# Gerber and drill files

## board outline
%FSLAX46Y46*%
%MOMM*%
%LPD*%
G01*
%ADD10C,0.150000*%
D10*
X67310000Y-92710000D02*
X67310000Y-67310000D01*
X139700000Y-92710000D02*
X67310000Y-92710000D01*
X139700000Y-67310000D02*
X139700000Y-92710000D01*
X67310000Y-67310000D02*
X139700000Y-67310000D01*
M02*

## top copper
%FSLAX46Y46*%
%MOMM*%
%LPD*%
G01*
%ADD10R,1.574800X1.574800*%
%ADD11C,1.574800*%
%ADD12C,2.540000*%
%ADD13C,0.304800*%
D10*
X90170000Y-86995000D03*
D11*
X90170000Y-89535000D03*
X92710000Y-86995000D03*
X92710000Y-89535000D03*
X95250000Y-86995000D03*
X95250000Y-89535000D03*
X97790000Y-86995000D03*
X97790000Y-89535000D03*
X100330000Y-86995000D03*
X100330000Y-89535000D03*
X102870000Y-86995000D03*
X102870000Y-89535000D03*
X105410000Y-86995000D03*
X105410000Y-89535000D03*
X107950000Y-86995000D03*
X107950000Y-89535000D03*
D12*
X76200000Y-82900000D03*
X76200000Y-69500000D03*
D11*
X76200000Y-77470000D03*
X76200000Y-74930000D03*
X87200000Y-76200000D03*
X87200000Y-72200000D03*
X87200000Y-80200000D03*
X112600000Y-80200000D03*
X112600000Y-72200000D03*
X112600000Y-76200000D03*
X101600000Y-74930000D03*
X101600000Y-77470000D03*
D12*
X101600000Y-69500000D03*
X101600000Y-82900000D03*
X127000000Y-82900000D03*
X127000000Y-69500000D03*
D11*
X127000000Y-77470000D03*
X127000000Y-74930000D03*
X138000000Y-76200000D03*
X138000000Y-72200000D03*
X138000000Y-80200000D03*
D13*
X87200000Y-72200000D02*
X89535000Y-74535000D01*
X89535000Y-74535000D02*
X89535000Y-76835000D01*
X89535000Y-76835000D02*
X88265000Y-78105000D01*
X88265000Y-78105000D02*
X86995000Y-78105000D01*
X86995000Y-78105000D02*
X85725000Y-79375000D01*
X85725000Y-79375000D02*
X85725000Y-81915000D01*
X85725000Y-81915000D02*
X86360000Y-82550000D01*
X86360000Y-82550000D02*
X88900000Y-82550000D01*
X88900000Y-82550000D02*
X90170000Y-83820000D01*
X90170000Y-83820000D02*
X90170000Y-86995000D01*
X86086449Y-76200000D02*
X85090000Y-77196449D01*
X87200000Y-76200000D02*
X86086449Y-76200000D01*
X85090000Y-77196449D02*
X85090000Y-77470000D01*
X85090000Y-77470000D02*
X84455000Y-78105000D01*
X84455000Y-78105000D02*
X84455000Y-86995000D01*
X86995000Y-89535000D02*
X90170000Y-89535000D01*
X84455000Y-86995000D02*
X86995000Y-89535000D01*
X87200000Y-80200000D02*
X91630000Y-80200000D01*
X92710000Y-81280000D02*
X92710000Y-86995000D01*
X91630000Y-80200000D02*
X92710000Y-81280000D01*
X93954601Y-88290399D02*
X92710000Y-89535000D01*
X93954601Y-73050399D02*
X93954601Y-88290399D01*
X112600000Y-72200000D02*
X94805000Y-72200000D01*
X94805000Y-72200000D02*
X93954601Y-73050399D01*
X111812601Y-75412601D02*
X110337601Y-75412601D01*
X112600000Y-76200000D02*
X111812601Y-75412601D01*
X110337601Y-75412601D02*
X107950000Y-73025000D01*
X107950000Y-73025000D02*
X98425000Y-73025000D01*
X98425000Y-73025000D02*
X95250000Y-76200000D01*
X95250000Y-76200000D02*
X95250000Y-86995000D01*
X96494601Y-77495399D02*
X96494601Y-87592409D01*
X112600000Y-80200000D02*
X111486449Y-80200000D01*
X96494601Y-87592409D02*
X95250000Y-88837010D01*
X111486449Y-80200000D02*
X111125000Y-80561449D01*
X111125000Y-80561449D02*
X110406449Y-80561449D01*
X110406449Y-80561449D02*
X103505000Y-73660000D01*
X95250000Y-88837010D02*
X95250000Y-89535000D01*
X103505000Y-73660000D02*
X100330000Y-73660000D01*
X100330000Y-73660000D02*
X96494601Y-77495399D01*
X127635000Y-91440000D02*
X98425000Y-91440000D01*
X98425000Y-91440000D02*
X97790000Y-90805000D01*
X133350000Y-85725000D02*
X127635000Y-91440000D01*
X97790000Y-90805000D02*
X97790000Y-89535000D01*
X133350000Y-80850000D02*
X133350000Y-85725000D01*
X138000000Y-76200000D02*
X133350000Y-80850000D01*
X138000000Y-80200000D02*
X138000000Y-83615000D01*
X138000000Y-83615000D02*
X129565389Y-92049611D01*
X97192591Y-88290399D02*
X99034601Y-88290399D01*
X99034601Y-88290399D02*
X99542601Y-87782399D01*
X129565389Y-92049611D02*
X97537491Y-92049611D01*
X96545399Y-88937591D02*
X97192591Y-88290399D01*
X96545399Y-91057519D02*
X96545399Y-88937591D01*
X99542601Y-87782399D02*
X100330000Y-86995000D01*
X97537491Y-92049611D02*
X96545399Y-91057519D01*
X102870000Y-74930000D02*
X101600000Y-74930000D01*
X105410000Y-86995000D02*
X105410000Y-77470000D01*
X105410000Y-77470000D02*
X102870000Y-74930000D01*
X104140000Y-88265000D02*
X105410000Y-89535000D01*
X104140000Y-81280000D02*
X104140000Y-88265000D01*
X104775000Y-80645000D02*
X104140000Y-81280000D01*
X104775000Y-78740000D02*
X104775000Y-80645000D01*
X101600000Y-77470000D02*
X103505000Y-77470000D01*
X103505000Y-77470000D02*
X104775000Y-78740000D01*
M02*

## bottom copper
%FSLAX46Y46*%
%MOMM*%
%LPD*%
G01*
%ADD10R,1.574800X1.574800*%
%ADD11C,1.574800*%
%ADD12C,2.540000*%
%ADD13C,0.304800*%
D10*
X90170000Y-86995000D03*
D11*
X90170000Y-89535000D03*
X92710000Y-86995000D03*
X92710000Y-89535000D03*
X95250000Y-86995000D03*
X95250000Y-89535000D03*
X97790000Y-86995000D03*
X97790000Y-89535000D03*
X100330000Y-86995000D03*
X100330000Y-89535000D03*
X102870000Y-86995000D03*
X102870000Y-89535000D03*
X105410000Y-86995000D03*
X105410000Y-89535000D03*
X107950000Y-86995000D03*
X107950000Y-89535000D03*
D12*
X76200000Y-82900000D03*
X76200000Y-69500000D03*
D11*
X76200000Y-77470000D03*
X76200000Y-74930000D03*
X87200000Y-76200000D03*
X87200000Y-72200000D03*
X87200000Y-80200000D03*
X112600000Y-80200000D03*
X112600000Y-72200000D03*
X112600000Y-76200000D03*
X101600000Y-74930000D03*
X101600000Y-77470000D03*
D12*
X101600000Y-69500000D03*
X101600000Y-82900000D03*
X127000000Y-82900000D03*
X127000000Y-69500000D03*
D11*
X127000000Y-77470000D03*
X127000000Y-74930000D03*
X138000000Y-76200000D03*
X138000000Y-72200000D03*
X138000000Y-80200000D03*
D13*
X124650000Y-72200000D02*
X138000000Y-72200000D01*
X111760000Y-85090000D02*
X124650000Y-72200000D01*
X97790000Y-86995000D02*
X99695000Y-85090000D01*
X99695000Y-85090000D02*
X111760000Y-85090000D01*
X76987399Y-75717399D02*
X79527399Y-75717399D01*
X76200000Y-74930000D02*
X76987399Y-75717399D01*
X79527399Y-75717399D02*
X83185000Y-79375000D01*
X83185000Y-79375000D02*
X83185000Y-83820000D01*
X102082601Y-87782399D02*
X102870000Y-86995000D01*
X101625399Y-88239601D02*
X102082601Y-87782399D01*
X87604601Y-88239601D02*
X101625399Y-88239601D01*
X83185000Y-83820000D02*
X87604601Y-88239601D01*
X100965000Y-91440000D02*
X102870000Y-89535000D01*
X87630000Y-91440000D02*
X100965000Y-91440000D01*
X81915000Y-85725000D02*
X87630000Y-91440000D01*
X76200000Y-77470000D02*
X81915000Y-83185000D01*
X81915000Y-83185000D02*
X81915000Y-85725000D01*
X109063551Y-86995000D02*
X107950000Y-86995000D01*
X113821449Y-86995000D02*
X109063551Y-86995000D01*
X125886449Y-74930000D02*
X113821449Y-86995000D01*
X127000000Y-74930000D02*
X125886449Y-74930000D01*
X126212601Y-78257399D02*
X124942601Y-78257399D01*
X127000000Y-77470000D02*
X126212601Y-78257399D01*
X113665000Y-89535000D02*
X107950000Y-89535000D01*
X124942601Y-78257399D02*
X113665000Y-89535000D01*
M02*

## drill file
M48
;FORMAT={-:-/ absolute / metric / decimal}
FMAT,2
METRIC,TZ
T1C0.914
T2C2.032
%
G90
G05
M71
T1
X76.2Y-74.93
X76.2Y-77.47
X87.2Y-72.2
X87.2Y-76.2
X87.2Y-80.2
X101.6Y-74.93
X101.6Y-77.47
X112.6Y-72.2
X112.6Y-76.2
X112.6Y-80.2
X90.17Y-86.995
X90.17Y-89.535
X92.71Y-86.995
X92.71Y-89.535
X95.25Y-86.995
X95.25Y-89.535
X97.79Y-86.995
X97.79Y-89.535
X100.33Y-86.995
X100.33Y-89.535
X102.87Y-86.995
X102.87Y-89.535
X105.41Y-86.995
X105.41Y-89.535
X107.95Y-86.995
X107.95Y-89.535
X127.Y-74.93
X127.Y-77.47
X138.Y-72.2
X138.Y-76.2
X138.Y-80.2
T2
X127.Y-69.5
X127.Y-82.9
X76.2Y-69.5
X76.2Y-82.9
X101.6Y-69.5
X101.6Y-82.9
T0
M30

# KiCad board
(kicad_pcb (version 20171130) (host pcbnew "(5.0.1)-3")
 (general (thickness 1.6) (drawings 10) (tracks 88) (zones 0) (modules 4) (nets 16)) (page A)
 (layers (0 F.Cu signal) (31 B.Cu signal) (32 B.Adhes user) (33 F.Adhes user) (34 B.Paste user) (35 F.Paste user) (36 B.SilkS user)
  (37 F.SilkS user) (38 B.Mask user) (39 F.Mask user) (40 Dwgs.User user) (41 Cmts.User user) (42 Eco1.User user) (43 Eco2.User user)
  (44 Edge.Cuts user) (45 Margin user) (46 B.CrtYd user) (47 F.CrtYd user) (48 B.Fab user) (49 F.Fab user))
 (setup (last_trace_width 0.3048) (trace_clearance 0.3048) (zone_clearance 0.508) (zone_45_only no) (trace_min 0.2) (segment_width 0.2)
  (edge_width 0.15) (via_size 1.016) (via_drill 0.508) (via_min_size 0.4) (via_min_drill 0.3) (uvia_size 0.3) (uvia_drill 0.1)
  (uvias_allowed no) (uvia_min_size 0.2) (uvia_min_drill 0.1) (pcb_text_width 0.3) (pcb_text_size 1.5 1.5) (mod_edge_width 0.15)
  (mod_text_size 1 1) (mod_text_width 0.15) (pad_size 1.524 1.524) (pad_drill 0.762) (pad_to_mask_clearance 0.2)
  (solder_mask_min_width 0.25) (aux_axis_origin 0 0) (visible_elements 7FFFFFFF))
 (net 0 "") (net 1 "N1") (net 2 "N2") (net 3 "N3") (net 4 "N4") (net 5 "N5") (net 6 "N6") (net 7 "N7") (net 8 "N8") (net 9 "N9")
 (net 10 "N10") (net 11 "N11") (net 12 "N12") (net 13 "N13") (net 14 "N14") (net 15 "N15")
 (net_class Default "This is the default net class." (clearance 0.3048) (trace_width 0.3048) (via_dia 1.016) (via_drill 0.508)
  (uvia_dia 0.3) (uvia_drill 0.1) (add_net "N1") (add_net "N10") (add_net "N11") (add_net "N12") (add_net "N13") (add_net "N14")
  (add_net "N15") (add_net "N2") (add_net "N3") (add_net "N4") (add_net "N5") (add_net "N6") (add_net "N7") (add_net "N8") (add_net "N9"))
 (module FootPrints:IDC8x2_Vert (layer B.Cu) (at 99.06 88.265 180)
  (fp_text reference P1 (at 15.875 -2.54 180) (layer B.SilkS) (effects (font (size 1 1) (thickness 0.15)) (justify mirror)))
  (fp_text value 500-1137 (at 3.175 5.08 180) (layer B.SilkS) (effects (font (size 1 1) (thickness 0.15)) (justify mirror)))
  (pad 1 thru_hole rect (at 8.89 1.27 180) (size 1.5748 1.5748) (drill 0.9144) (layers *.Cu *.Mask B.SilkS) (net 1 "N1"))
  (pad 2 thru_hole circle (at 8.89 -1.27 180) (size 1.5748 1.5748) (drill 0.9144) (layers *.Cu *.Mask B.SilkS) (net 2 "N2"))
  (pad 3 thru_hole circle (at 6.35 1.27 180) (size 1.5748 1.5748) (drill 0.9144) (layers *.Cu *.Mask B.SilkS) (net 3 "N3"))
  (pad 4 thru_hole circle (at 6.35 -1.27 180) (size 1.5748 1.5748) (drill 0.9144) (layers *.Cu *.Mask B.SilkS) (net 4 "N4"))
  (pad 5 thru_hole circle (at 3.81 1.27 180) (size 1.5748 1.5748) (drill 0.9144) (layers *.Cu *.Mask B.SilkS) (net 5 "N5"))
  (pad 6 thru_hole circle (at 3.81 -1.27 180) (size 1.5748 1.5748) (drill 0.9144) (layers *.Cu *.Mask B.SilkS) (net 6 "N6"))
  (pad 7 thru_hole circle (at 1.27 1.27 180) (size 1.5748 1.5748) (drill 0.9144) (layers *.Cu *.Mask B.SilkS) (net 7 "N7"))
  (pad 8 thru_hole circle (at 1.27 -1.27 180) (size 1.5748 1.5748) (drill 0.9144) (layers *.Cu *.Mask B.SilkS) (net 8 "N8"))
  (pad 9 thru_hole circle (at -1.27 1.27 180) (size 1.5748 1.5748) (drill 0.9144) (layers *.Cu *.Mask B.SilkS) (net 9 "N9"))
  (pad 10 thru_hole circle (at -1.27 -1.27 180) (size 1.5748 1.5748) (drill 0.9144) (layers *.Cu *.Mask B.SilkS))
  (pad 11 thru_hole circle (at -3.81 1.27 180) (size 1.5748 1.5748) (drill 0.9144) (layers *.Cu *.Mask B.SilkS) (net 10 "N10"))
  (pad 12 thru_hole circle (at -3.81 -1.27 180) (size 1.5748 1.5748) (drill 0.9144) (layers *.Cu *.Mask B.SilkS) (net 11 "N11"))
  (pad 13 thru_hole circle (at -6.35 1.27 180) (size 1.5748 1.5748) (drill 0.9144) (layers *.Cu *.Mask B.SilkS) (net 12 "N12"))
  (pad 14 thru_hole circle (at -6.35 -1.27 180) (size 1.5748 1.5748) (drill 0.9144) (layers *.Cu *.Mask B.SilkS) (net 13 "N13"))
  (pad 15 thru_hole circle (at -8.89 1.27 180) (size 1.5748 1.5748) (drill 0.9144) (layers *.Cu *.Mask B.SilkS) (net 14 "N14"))
  (pad 16 thru_hole circle (at -8.89 -1.27 180) (size 1.5748 1.5748) (drill 0.9144) (layers *.Cu *.Mask B.SilkS) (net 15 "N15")))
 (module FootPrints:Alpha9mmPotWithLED (layer F.Cu) (at 76.2 76.2 90)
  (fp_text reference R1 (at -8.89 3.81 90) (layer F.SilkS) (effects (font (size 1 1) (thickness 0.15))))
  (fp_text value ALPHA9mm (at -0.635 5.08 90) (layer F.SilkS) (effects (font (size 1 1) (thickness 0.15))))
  (pad "" thru_hole circle (at -6.7 0 90) (size 2.54 2.54) (drill 2.032) (layers *.Cu *.Mask F.SilkS))
  (pad "" thru_hole circle (at 6.7 0 90) (size 2.54 2.54) (drill 2.032) (layers *.Cu *.Mask F.SilkS))
  (pad 4 thru_hole circle (at -1.27 0 90) (size 1.5748 1.5748) (drill 0.9144) (layers *.Cu *.Mask F.SilkS) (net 11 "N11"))
  (pad 5 thru_hole circle (at 1.27 0 90) (size 1.5748 1.5748) (drill 0.9144) (layers *.Cu *.Mask F.SilkS) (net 10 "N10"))
  (pad 2 thru_hole circle (at 0 11 90) (size 1.5748 1.5748) (drill 0.9144) (layers *.Cu *.Mask F.SilkS) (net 2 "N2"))
  (pad 3 thru_hole circle (at 4 11 90) (size 1.5748 1.5748) (drill 0.9144) (layers *.Cu *.Mask F.SilkS) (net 1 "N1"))
  (pad 1 thru_hole circle (at -4 11 90) (size 1.5748 1.5748) (drill 0.9144) (layers *.Cu *.Mask F.SilkS) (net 3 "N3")))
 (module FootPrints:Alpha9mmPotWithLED (layer F.Cu) (at 101.6 76.2 90)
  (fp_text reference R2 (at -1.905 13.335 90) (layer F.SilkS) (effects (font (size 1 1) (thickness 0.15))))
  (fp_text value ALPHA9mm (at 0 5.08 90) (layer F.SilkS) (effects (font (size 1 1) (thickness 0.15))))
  (pad 1 thru_hole circle (at -4 11 90) (size 1.5748 1.5748) (drill 0.9144) (layers *.Cu *.Mask F.SilkS) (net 6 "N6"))
  (pad 3 thru_hole circle (at 4 11 90) (size 1.5748 1.5748) (drill 0.9144) (layers *.Cu *.Mask F.SilkS) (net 4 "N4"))
  (pad 2 thru_hole circle (at 0 11 90) (size 1.5748 1.5748) (drill 0.9144) (layers *.Cu *.Mask F.SilkS) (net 5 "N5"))
  (pad 5 thru_hole circle (at 1.27 0 90) (size 1.5748 1.5748) (drill 0.9144) (layers *.Cu *.Mask F.SilkS) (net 12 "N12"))
  (pad 4 thru_hole circle (at -1.27 0 90) (size 1.5748 1.5748) (drill 0.9144) (layers *.Cu *.Mask F.SilkS) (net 13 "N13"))
  (pad "" thru_hole circle (at 6.7 0 90) (size 2.54 2.54) (drill 2.032) (layers *.Cu *.Mask F.SilkS))
  (pad "" thru_hole circle (at -6.7 0 90) (size 2.54 2.54) (drill 2.032) (layers *.Cu *.Mask F.SilkS)))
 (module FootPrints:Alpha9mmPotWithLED (layer F.Cu) (at 127 76.2 90)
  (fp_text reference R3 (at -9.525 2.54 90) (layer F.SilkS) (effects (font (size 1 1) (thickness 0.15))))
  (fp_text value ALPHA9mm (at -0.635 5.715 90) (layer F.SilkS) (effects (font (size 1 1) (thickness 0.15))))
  (pad "" thru_hole circle (at -6.7 0 90) (size 2.54 2.54) (drill 2.032) (layers *.Cu *.Mask F.SilkS))
  (pad "" thru_hole circle (at 6.7 0 90) (size 2.54 2.54) (drill 2.032) (layers *.Cu *.Mask F.SilkS))
  (pad 4 thru_hole circle (at -1.27 0 90) (size 1.5748 1.5748) (drill 0.9144) (layers *.Cu *.Mask F.SilkS) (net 15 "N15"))
  (pad 5 thru_hole circle (at 1.27 0 90) (size 1.5748 1.5748) (drill 0.9144) (layers *.Cu *.Mask F.SilkS) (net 14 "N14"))
  (pad 2 thru_hole circle (at 0 11 90) (size 1.5748 1.5748) (drill 0.9144) (layers *.Cu *.Mask F.SilkS) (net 8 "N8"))
  (pad 3 thru_hole circle (at 4 11 90) (size 1.5748 1.5748) (drill 0.9144) (layers *.Cu *.Mask F.SilkS) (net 7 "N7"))
  (pad 1 thru_hole circle (at -4 11 90) (size 1.5748 1.5748) (drill 0.9144) (layers *.Cu *.Mask F.SilkS) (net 9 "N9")))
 (gr_line (start 67.31 92.71) (end 67.31 67.31) (layer Edge.Cuts) (width 0.15))
 (gr_line (start 139.7 92.71) (end 67.31 92.71) (layer Edge.Cuts) (width 0.15))
 (gr_line (start 139.7 67.31) (end 139.7 92.71) (layer Edge.Cuts) (width 0.15))
 (gr_line (start 67.31 67.31) (end 139.7 67.31) (layer Edge.Cuts) (width 0.15))
 (segment (start 87.2 72.2) (end 89.535 74.535) (width 0.3048) (layer F.Cu) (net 1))
 (segment (start 89.535 74.535) (end 89.535 76.835) (width 0.3048) (layer F.Cu) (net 1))
 (segment (start 89.535 76.835) (end 88.265 78.105) (width 0.3048) (layer F.Cu) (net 1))
 (segment (start 88.265 78.105) (end 86.995 78.105) (width 0.3048) (layer F.Cu) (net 1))
 (segment (start 86.995 78.105) (end 85.725 79.375) (width 0.3048) (layer F.Cu) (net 1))
 (segment (start 85.725 79.375) (end 85.725 81.915) (width 0.3048) (layer F.Cu) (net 1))
 (segment (start 85.725 81.915) (end 86.36 82.55) (width 0.3048) (layer F.Cu) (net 1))
 (segment (start 86.36 82.55) (end 88.9 82.55) (width 0.3048) (layer F.Cu) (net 1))
 (segment (start 88.9 82.55) (end 90.17 83.82) (width 0.3048) (layer F.Cu) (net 1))
 (segment (start 90.17 83.82) (end 90.17 86.995) (width 0.3048) (layer F.Cu) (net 1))
 (segment (start 86.086449 76.2) (end 85.09 77.196449) (width 0.3048) (layer F.Cu) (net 2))
 (segment (start 87.2 76.2) (end 86.086449 76.2) (width 0.3048) (layer F.Cu) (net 2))
 (segment (start 85.09 77.196449) (end 85.09 77.47) (width 0.3048) (layer F.Cu) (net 2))
 (segment (start 85.09 77.47) (end 84.455 78.105) (width 0.3048) (layer F.Cu) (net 2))
 (segment (start 84.455 78.105) (end 84.455 86.995) (width 0.3048) (layer F.Cu) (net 2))
 (segment (start 86.995 89.535) (end 90.17 89.535) (width 0.3048) (layer F.Cu) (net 2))
 (segment (start 84.455 86.995) (end 86.995 89.535) (width 0.3048) (layer F.Cu) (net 2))
 (segment (start 87.2 80.2) (end 91.63 80.2) (width 0.3048) (layer F.Cu) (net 3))
 (segment (start 92.71 81.28) (end 92.71 86.995) (width 0.3048) (layer F.Cu) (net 3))
 (segment (start 91.63 80.2) (end 92.71 81.28) (width 0.3048) (layer F.Cu) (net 3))
 (segment (start 93.954601 88.290399) (end 92.71 89.535) (width 0.3048) (layer F.Cu) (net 4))
 (segment (start 93.954601 73.050399) (end 93.954601 88.290399) (width 0.3048) (layer F.Cu) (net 4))
 (segment (start 112.6 72.2) (end 94.805 72.2) (width 0.3048) (layer F.Cu) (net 4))
 (segment (start 94.805 72.2) (end 93.954601 73.050399) (width 0.3048) (layer F.Cu) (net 4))
 (segment (start 111.812601 75.412601) (end 110.337601 75.412601) (width 0.3048) (layer F.Cu) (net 5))
 (segment (start 112.6 76.2) (end 111.812601 75.412601) (width 0.3048) (layer F.Cu) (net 5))
 (segment (start 110.337601 75.412601) (end 107.95 73.025) (width 0.3048) (layer F.Cu) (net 5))
 (segment (start 107.95 73.025) (end 98.425 73.025) (width 0.3048) (layer F.Cu) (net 5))
 (segment (start 98.425 73.025) (end 95.25 76.2) (width 0.3048) (layer F.Cu) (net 5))
 (segment (start 95.25 76.2) (end 95.25 86.995) (width 0.3048) (layer F.Cu) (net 5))
 (segment (start 96.494601 77.495399) (end 96.494601 87.592409) (width 0.3048) (layer F.Cu) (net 6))
 (segment (start 112.6 80.2) (end 111.486449 80.2) (width 0.3048) (layer F.Cu) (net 6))
 (segment (start 96.494601 87.592409) (end 95.25 88.83701) (width 0.3048) (layer F.Cu) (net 6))
 (segment (start 111.486449 80.2) (end 111.125 80.561449) (width 0.3048) (layer F.Cu) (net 6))
 (segment (start 111.125 80.561449) (end 110.406449 80.561449) (width 0.3048) (layer F.Cu) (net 6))
 (segment (start 110.406449 80.561449) (end 103.505 73.66) (width 0.3048) (layer F.Cu) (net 6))
 (segment (start 95.25 88.83701) (end 95.25 89.535) (width 0.3048) (layer F.Cu) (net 6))
 (segment (start 103.505 73.66) (end 100.33 73.66) (width 0.3048) (layer F.Cu) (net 6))
 (segment (start 100.33 73.66) (end 96.494601 77.495399) (width 0.3048) (layer F.Cu) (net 6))
 (segment (start 124.65 72.2) (end 138 72.2) (width 0.3048) (layer B.Cu) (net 7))
 (segment (start 111.76 85.09) (end 124.65 72.2) (width 0.3048) (layer B.Cu) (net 7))
 (segment (start 97.79 86.995) (end 99.695 85.09) (width 0.3048) (layer B.Cu) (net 7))
 (segment (start 99.695 85.09) (end 111.76 85.09) (width 0.3048) (layer B.Cu) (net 7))
 (segment (start 127.635 91.44) (end 98.425 91.44) (width 0.3048) (layer F.Cu) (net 8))
 (segment (start 98.425 91.44) (end 97.79 90.805) (width 0.3048) (layer F.Cu) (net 8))
 (segment (start 133.35 85.725) (end 127.635 91.44) (width 0.3048) (layer F.Cu) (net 8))
 (segment (start 97.79 90.805) (end 97.79 89.535) (width 0.3048) (layer F.Cu) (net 8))
 (segment (start 133.35 80.85) (end 133.35 85.725) (width 0.3048) (layer F.Cu) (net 8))
 (segment (start 138 76.2) (end 133.35 80.85) (width 0.3048) (layer F.Cu) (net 8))
 (segment (start 138 80.2) (end 138 83.615) (width 0.3048) (layer F.Cu) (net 9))
 (segment (start 138 83.615) (end 129.565389 92.049611) (width 0.3048) (layer F.Cu) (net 9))
 (segment (start 97.192591 88.290399) (end 99.034601 88.290399) (width 0.3048) (layer F.Cu) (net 9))
 (segment (start 99.034601 88.290399) (end 99.542601 87.782399) (width 0.3048) (layer F.Cu) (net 9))
 (segment (start 129.565389 92.049611) (end 97.537491 92.049611) (width 0.3048) (layer F.Cu) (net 9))
 (segment (start 96.545399 88.937591) (end 97.192591 88.290399) (width 0.3048) (layer F.Cu) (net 9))
 (segment (start 96.545399 91.057519) (end 96.545399 88.937591) (width 0.3048) (layer F.Cu) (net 9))
 (segment (start 99.542601 87.782399) (end 100.33 86.995) (width 0.3048) (layer F.Cu) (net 9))
 (segment (start 97.537491 92.049611) (end 96.545399 91.057519) (width 0.3048) (layer F.Cu) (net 9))
 (segment (start 76.987399 75.717399) (end 79.527399 75.717399) (width 0.3048) (layer B.Cu) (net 10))
 (segment (start 76.2 74.93) (end 76.987399 75.717399) (width 0.3048) (layer B.Cu) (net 10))
 (segment (start 79.527399 75.717399) (end 83.185 79.375) (width 0.3048) (layer B.Cu) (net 10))
 (segment (start 83.185 79.375) (end 83.185 83.82) (width 0.3048) (layer B.Cu) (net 10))
 (segment (start 102.082601 87.782399) (end 102.87 86.995) (width 0.3048) (layer B.Cu) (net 10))
 (segment (start 101.625399 88.239601) (end 102.082601 87.782399) (width 0.3048) (layer B.Cu) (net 10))
 (segment (start 87.604601 88.239601) (end 101.625399 88.239601) (width 0.3048) (layer B.Cu) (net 10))
 (segment (start 83.185 83.82) (end 87.604601 88.239601) (width 0.3048) (layer B.Cu) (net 10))
 (segment (start 100.965 91.44) (end 102.87 89.535) (width 0.3048) (layer B.Cu) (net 11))
 (segment (start 87.63 91.44) (end 100.965 91.44) (width 0.3048) (layer B.Cu) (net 11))
 (segment (start 81.915 85.725) (end 87.63 91.44) (width 0.3048) (layer B.Cu) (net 11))
 (segment (start 76.2 77.47) (end 81.915 83.185) (width 0.3048) (layer B.Cu) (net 11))
 (segment (start 81.915 83.185) (end 81.915 85.725) (width 0.3048) (layer B.Cu) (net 11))
 (segment (start 102.87 74.93) (end 101.6 74.93) (width 0.3048) (layer F.Cu) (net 12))
 (segment (start 105.41 86.995) (end 105.41 77.47) (width 0.3048) (layer F.Cu) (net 12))
 (segment (start 105.41 77.47) (end 102.87 74.93) (width 0.3048) (layer F.Cu) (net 12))
 (segment (start 104.14 88.265) (end 105.41 89.535) (width 0.3048) (layer F.Cu) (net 13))
 (segment (start 104.14 81.28) (end 104.14 88.265) (width 0.3048) (layer F.Cu) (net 13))
 (segment (start 104.775 80.645) (end 104.14 81.28) (width 0.3048) (layer F.Cu) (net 13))
 (segment (start 104.775 78.74) (end 104.775 80.645) (width 0.3048) (layer F.Cu) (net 13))
 (segment (start 101.6 77.47) (end 103.505 77.47) (width 0.3048) (layer F.Cu) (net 13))
 (segment (start 103.505 77.47) (end 104.775 78.74) (width 0.3048) (layer F.Cu) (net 13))
 (segment (start 109.063551 86.995) (end 107.95 86.995) (width 0.3048) (layer B.Cu) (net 14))
 (segment (start 113.821449 86.995) (end 109.063551 86.995) (width 0.3048) (layer B.Cu) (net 14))
 (segment (start 125.886449 74.93) (end 113.821449 86.995) (width 0.3048) (layer B.Cu) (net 14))
 (segment (start 127 74.93) (end 125.886449 74.93) (width 0.3048) (layer B.Cu) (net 14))
 (segment (start 126.212601 78.257399) (end 124.942601 78.257399) (width 0.3048) (layer B.Cu) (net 15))
 (segment (start 127 77.47) (end 126.212601 78.257399) (width 0.3048) (layer B.Cu) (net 15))
 (segment (start 113.665 89.535) (end 107.95 89.535) (width 0.3048) (layer B.Cu) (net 15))
 (segment (start 124.942601 78.257399) (end 113.665 89.535) (width 0.3048) (layer B.Cu) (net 15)))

